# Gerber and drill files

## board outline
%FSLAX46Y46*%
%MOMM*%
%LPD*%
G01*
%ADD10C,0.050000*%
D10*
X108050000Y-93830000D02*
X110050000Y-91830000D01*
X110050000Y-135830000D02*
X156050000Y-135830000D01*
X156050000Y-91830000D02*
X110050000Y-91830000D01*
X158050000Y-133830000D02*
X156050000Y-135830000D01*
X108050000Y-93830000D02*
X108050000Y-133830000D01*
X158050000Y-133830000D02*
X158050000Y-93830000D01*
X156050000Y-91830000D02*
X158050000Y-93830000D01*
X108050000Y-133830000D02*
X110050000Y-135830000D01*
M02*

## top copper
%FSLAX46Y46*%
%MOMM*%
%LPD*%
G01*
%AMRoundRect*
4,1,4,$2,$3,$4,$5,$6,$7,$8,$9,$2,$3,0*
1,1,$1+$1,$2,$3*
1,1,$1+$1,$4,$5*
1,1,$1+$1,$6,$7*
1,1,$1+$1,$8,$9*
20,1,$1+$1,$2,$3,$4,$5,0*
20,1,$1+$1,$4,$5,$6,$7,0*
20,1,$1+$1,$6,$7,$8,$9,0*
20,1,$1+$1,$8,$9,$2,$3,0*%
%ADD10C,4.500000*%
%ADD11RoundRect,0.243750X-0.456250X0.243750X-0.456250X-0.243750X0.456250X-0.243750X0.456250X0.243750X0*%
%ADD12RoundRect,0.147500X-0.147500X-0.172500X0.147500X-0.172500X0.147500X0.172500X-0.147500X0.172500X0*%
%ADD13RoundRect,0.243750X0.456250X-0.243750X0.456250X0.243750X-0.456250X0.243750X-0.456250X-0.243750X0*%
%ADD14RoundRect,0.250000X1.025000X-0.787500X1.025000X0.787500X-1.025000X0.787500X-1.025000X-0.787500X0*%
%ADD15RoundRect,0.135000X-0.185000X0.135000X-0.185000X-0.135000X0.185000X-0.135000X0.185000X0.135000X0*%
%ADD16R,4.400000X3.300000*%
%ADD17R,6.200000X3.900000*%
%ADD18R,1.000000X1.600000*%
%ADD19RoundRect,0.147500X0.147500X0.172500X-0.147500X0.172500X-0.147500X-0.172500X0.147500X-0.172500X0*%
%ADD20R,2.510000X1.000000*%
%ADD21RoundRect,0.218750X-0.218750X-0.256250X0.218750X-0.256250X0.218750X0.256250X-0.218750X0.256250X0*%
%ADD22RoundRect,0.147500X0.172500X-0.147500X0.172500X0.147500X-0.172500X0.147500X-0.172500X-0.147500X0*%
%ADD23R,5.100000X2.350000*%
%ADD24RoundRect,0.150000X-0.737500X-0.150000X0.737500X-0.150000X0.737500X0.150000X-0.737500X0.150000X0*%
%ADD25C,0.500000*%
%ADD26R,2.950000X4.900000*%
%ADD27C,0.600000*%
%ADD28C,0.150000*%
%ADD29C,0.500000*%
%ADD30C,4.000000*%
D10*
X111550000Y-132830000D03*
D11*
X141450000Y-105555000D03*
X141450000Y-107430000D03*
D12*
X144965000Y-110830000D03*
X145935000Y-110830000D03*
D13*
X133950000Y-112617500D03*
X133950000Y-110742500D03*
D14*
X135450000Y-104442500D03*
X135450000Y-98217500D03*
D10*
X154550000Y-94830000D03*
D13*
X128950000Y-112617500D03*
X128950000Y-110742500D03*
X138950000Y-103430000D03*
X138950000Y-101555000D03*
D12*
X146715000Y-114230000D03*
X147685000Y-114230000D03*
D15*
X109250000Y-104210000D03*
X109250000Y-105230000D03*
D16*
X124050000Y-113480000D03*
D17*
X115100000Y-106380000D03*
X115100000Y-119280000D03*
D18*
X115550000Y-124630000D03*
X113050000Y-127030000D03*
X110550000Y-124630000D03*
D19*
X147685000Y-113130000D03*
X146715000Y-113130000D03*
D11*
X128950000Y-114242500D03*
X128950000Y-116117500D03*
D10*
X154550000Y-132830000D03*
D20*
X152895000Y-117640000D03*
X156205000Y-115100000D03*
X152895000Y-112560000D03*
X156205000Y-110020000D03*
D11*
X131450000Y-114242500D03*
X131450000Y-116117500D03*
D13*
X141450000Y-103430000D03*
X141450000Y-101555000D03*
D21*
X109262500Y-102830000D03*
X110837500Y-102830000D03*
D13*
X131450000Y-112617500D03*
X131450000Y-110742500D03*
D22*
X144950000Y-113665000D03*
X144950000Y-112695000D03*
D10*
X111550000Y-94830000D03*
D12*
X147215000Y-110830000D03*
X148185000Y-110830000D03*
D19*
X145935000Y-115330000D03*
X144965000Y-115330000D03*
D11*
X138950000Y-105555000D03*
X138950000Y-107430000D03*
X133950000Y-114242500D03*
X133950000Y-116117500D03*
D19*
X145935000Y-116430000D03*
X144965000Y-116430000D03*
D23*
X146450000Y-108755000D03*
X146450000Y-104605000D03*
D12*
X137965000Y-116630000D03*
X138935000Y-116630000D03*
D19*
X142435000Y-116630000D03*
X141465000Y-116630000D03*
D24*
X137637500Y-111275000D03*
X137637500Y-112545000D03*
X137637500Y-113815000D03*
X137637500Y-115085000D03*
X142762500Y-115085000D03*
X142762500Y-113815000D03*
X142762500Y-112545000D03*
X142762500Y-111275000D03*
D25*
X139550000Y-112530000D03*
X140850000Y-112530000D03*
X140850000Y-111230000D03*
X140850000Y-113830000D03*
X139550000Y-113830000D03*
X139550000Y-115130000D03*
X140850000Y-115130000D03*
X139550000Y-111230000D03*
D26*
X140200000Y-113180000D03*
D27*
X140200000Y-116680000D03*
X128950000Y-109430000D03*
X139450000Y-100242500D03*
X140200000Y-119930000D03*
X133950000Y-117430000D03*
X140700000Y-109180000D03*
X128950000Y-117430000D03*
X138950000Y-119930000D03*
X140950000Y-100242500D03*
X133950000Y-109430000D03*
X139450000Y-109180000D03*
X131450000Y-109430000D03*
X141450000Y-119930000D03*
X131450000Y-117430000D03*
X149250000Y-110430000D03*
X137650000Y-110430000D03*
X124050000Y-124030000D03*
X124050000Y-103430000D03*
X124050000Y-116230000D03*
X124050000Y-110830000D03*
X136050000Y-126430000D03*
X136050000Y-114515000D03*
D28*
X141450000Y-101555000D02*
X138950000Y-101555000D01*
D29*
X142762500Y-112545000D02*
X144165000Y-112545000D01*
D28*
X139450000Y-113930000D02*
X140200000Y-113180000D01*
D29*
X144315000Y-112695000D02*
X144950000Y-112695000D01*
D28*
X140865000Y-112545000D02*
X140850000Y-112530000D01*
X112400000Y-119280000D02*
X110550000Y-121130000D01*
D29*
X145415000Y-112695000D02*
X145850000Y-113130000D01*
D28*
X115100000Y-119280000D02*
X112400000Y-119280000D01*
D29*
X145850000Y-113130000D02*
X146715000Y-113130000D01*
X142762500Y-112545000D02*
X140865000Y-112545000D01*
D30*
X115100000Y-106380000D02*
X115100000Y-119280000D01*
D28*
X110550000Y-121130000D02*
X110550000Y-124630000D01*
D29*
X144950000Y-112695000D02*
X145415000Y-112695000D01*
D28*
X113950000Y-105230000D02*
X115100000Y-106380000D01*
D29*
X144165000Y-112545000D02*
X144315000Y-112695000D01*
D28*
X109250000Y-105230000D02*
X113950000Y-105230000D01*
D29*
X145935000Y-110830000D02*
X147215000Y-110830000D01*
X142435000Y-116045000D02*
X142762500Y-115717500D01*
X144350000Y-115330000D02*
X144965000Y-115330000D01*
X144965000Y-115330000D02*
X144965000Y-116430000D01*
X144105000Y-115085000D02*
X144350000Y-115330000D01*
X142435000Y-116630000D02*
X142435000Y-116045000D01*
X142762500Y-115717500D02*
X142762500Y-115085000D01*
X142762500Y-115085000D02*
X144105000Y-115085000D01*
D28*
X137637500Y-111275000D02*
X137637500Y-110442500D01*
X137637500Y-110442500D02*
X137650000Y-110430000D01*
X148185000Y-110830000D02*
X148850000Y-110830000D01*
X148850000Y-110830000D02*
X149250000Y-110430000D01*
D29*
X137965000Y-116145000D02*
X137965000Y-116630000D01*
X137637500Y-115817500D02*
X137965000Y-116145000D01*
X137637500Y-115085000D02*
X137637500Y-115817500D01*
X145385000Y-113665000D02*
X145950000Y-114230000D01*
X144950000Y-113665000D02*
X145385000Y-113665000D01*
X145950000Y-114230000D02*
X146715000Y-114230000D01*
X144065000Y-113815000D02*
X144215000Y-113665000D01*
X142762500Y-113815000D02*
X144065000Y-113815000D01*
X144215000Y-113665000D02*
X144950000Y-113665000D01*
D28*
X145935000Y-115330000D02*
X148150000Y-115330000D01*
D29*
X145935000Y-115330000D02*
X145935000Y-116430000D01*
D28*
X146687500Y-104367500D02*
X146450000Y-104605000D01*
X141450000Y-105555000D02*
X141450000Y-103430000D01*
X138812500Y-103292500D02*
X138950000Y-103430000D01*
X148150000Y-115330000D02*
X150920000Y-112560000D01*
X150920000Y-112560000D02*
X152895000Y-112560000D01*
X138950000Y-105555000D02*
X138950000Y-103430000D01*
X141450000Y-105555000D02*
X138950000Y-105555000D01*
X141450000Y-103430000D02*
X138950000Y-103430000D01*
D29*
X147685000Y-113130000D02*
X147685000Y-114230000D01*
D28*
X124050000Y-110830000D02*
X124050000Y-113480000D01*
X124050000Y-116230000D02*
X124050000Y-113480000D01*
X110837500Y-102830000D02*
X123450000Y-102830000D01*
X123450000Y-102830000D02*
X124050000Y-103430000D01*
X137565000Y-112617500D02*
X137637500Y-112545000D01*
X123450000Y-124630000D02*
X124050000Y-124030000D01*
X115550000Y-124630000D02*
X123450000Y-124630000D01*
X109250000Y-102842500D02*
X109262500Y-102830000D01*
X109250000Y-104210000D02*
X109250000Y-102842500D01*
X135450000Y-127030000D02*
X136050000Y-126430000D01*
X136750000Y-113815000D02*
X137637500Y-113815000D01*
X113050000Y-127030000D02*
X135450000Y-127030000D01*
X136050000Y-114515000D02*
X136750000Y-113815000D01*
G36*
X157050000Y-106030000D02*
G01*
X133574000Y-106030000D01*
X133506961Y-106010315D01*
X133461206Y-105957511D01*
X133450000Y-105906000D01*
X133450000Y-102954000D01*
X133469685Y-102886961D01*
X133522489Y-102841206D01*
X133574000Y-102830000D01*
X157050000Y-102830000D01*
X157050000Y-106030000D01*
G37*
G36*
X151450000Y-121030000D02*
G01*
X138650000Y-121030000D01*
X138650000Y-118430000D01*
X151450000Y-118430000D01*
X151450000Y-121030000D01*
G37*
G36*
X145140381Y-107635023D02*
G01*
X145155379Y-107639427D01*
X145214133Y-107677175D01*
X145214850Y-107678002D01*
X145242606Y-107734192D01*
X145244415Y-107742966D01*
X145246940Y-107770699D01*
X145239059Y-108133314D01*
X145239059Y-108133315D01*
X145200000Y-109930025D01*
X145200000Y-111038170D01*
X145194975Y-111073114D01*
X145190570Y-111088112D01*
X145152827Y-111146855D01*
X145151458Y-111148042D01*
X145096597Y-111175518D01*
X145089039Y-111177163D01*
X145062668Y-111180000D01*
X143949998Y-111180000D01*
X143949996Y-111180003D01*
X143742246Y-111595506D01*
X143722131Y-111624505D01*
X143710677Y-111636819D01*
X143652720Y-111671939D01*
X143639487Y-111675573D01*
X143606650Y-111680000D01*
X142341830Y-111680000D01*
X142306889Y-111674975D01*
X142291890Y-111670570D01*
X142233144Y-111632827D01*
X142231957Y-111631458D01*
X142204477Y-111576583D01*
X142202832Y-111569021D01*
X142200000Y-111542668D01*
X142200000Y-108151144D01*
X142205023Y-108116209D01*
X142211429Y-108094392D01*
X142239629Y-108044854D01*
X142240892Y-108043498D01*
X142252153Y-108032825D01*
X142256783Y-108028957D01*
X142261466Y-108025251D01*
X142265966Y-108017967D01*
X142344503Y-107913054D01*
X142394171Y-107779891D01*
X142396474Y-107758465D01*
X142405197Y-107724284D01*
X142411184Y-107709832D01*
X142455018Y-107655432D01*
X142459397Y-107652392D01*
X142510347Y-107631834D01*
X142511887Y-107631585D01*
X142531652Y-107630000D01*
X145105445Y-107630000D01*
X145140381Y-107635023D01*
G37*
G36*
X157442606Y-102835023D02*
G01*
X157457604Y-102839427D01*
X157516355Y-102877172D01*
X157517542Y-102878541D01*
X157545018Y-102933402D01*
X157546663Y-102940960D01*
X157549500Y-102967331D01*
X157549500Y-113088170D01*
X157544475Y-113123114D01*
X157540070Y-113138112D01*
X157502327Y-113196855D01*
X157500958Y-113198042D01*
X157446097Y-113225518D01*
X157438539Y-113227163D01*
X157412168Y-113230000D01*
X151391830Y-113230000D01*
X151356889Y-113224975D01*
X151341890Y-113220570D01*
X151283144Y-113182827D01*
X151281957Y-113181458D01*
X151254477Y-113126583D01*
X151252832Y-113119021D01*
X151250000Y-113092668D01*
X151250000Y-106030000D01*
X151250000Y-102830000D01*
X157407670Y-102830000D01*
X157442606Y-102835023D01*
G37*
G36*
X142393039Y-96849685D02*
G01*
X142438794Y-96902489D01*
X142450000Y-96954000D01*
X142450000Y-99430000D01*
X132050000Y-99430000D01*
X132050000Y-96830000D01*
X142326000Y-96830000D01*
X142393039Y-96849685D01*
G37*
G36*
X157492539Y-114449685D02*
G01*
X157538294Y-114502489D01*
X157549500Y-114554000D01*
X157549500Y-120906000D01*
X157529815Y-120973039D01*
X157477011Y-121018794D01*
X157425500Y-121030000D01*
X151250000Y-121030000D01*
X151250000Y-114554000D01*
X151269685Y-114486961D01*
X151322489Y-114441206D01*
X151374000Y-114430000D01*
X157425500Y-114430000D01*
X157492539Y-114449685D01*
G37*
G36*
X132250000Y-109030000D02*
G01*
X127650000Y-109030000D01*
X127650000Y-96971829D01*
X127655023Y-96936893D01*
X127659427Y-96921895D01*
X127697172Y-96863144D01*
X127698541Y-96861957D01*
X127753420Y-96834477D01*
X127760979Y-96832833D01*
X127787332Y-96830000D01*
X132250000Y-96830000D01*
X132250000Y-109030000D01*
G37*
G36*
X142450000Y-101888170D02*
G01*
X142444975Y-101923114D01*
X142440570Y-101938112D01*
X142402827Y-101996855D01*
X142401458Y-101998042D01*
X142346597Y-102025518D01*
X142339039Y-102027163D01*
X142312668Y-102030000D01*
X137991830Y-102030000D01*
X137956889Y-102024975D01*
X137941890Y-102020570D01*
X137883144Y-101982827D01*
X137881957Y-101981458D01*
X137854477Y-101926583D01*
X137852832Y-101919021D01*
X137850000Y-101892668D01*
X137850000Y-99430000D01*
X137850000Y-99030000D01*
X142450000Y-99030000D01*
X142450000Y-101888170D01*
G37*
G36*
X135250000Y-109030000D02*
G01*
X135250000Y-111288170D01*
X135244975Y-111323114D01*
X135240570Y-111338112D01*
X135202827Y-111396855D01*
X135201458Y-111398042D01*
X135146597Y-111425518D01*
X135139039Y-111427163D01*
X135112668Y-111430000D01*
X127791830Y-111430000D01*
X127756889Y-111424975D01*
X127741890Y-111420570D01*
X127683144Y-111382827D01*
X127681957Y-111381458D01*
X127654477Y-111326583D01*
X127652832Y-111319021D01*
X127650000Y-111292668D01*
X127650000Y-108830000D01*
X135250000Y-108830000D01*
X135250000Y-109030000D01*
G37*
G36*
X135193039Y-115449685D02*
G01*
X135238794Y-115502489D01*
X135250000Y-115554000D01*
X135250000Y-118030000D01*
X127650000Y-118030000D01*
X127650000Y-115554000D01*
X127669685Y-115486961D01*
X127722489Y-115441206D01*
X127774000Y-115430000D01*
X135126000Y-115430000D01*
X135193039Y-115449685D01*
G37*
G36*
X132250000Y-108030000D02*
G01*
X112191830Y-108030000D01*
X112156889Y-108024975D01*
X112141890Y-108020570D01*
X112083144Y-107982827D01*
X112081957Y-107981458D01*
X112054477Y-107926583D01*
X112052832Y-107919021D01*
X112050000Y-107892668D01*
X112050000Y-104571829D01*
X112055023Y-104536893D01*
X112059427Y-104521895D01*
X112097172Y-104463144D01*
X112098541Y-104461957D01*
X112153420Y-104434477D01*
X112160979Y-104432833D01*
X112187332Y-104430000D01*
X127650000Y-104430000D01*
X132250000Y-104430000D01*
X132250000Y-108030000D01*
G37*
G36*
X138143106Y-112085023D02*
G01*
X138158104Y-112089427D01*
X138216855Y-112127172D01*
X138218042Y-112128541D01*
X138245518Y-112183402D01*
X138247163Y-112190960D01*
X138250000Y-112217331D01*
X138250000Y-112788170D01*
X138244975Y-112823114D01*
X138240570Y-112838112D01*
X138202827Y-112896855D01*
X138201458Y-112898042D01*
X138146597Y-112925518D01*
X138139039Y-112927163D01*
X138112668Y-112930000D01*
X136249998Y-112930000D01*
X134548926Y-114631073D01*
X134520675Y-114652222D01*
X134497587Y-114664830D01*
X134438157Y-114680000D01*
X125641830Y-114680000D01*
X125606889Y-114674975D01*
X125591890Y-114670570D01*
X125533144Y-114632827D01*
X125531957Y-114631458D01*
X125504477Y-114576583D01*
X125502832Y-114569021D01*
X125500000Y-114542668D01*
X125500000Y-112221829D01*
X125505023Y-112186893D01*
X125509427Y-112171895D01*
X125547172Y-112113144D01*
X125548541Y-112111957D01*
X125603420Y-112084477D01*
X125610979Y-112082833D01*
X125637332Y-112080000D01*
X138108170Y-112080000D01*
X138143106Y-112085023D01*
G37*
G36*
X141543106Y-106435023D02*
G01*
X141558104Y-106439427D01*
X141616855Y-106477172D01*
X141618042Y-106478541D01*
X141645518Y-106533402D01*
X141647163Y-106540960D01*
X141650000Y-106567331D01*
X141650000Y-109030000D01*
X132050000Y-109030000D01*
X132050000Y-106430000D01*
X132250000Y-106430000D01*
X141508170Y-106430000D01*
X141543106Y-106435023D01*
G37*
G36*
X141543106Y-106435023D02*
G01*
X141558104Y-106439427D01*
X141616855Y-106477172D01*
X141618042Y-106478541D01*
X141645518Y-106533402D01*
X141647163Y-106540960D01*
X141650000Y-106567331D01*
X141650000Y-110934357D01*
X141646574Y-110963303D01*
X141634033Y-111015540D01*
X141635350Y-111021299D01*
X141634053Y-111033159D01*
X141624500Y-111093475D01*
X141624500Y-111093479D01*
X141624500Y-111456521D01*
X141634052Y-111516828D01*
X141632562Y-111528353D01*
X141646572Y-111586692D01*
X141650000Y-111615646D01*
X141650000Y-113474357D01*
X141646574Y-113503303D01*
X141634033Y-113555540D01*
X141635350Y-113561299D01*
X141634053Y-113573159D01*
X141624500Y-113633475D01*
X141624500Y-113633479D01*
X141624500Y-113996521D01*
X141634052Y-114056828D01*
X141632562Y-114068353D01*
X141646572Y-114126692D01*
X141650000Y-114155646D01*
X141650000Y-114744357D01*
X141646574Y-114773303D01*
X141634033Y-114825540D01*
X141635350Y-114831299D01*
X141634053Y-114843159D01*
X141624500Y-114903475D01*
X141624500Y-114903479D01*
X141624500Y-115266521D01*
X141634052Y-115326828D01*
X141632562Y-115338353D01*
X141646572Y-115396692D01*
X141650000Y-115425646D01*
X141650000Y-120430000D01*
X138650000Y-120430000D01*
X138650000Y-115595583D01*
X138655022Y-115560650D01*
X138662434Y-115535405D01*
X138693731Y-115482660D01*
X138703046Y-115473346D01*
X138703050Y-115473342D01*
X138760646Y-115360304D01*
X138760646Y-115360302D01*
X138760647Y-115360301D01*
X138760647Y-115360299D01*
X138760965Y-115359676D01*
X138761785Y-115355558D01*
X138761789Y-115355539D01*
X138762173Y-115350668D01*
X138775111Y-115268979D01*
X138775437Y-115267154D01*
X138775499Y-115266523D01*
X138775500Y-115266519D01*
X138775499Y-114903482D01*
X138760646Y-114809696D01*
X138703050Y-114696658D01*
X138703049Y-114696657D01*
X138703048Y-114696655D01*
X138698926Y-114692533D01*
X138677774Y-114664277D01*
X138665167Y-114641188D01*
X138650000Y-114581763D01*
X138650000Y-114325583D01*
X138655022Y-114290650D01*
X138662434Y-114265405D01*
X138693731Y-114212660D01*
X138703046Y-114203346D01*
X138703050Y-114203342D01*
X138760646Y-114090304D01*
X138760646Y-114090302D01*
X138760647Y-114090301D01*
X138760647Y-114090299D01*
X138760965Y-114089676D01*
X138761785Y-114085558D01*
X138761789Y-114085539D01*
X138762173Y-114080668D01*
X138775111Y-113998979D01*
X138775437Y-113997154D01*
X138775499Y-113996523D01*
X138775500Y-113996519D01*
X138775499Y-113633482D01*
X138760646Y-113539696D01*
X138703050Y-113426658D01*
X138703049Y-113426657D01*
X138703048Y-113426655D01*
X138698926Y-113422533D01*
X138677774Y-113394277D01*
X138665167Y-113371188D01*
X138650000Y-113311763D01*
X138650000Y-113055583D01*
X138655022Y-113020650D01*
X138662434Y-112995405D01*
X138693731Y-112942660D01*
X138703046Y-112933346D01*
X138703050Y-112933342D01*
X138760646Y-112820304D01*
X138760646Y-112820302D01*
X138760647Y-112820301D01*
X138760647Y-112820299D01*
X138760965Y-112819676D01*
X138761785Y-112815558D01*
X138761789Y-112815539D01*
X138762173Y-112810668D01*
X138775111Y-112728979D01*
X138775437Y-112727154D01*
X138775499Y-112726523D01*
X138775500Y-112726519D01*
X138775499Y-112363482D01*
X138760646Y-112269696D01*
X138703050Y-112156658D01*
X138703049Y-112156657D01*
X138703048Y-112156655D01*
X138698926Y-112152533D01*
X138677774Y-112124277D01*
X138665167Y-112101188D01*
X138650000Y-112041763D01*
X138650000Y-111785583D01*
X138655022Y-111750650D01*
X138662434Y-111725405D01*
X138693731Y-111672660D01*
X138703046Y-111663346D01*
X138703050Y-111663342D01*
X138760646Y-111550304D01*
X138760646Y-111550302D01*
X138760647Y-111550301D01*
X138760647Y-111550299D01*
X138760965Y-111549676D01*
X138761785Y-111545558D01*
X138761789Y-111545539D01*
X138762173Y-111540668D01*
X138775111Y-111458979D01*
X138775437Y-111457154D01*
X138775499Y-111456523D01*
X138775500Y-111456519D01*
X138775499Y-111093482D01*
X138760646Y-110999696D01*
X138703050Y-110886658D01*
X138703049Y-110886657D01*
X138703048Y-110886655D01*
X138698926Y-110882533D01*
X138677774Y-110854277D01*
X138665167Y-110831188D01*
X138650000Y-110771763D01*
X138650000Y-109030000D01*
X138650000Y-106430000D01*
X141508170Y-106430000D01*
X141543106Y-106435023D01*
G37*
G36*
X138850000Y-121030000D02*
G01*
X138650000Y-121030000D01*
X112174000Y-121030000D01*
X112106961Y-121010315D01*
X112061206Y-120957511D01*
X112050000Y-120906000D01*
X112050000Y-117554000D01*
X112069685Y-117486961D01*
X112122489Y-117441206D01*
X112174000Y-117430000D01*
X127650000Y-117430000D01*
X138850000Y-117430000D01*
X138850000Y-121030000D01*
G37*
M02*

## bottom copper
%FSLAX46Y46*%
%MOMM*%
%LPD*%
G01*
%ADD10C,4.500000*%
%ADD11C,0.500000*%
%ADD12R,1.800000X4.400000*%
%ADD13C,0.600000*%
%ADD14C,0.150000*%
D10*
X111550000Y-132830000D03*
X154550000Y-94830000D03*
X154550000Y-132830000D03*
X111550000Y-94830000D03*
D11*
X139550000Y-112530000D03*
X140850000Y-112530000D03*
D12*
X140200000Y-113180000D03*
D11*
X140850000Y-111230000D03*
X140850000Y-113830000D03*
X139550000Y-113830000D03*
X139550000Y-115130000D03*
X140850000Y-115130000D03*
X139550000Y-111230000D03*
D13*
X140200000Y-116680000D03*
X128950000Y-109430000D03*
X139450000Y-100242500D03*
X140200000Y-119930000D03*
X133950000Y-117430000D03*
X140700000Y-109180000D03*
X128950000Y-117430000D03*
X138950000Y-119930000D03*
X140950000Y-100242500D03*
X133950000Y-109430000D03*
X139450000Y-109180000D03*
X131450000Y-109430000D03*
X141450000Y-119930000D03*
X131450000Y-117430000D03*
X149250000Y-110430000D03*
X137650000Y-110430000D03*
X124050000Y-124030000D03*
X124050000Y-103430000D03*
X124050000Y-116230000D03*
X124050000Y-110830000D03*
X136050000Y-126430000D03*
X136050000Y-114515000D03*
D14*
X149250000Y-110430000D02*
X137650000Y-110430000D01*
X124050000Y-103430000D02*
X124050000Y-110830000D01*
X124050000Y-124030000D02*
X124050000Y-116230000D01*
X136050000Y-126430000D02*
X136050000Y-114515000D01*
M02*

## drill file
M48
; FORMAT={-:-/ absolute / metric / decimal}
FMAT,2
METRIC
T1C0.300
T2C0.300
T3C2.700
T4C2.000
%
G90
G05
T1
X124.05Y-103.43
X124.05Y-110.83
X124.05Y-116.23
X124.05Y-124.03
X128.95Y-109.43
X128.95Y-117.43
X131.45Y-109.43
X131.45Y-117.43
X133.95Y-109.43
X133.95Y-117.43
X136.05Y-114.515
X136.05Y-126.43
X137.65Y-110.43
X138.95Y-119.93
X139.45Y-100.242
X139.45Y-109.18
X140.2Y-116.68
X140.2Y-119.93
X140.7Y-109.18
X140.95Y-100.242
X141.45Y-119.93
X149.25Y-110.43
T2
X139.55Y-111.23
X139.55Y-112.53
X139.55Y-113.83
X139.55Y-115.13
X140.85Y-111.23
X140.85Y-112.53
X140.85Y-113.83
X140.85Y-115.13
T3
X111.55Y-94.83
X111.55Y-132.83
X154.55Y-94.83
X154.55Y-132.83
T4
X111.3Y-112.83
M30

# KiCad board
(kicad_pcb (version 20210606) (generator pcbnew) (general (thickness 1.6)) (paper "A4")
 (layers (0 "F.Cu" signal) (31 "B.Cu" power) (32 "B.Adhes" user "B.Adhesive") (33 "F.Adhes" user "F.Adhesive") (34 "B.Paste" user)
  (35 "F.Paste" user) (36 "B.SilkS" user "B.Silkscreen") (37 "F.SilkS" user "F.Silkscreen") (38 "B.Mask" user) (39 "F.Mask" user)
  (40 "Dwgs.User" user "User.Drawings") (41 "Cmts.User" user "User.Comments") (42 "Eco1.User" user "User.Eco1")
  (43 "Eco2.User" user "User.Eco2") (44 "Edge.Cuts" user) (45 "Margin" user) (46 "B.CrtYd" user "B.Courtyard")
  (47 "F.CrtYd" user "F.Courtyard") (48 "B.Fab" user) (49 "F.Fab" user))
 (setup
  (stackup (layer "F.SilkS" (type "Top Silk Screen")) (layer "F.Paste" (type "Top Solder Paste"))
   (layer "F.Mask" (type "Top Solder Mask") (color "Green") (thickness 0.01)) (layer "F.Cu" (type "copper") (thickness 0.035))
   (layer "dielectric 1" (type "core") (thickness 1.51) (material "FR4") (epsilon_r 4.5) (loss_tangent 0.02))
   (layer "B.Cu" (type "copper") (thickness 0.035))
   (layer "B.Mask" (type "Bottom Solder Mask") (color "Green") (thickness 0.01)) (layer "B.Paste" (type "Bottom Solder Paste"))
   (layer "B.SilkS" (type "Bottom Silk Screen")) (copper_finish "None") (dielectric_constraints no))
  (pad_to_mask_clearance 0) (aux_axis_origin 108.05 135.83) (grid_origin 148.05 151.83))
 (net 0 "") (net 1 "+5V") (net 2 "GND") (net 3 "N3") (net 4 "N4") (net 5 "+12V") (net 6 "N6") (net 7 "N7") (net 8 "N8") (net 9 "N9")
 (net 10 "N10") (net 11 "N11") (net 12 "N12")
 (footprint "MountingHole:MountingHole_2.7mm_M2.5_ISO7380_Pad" (layer "F.Cu") (at 111.55 132.83)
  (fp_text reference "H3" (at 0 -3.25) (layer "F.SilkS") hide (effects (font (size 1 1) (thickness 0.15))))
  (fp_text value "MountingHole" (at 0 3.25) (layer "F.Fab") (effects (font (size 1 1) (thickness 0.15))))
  (pad "1" thru_hole circle locked (at 0 0) (size 4.5 4.5) (drill 2.7) (layers *.Cu *.Mask)))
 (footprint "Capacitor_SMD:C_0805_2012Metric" (layer "F.Cu") (at 141.45 106.4925 -90)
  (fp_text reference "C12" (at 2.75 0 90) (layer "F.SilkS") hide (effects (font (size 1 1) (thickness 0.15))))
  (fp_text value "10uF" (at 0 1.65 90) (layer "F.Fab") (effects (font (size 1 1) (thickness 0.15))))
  (pad "1" smd roundrect locked (at -0.9375 0 270) (size 0.975 1.4) (layers "F.Cu" "F.Paste" "F.Mask") (roundrect_rratio 0.25) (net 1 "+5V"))
  (pad "2" smd roundrect locked (at 0.9375 0 270) (size 0.975 1.4) (layers "F.Cu" "F.Paste" "F.Mask") (roundrect_rratio 0.25) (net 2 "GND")))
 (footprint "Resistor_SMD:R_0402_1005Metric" (layer "F.Cu") (at 145.45 110.83)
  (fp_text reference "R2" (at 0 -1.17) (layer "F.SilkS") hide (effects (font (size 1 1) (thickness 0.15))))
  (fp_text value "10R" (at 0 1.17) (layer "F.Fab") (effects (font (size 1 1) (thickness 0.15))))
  (pad "1" smd roundrect locked (at -0.485 0) (size 0.59 0.64) (layers "F.Cu" "F.Paste" "F.Mask") (roundrect_rratio 0.25) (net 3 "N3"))
  (pad "2" smd roundrect locked (at 0.485 0) (size 0.59 0.64) (layers "F.Cu" "F.Paste" "F.Mask") (roundrect_rratio 0.25) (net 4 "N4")))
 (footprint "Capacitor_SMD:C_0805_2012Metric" (layer "F.Cu") (at 133.95 111.68 90)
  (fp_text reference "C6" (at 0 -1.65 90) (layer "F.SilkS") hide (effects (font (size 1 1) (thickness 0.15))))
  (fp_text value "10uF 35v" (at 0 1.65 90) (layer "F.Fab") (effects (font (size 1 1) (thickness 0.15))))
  (pad "1" smd roundrect locked (at -0.9375 0 90) (size 0.975 1.4) (layers "F.Cu" "F.Paste" "F.Mask") (roundrect_rratio 0.25) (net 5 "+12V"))
  (pad "2" smd roundrect locked (at 0.9375 0 90) (size 0.975 1.4) (layers "F.Cu" "F.Paste" "F.Mask") (roundrect_rratio 0.25) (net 2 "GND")))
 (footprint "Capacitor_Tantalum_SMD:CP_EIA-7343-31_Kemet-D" (layer "F.Cu") (at 135.45 101.33 90)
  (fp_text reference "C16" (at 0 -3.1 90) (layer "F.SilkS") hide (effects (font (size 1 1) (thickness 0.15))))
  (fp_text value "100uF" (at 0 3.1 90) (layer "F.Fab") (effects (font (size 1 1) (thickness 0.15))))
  (pad "1" smd roundrect locked (at -3.1125 0 90) (size 2.075 2.55) (layers "F.Cu" "F.Paste" "F.Mask") (roundrect_rratio 0.1204819277)
   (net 1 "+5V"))
  (pad "2" smd roundrect locked (at 3.1125 0 90) (size 2.075 2.55) (layers "F.Cu" "F.Paste" "F.Mask") (roundrect_rratio 0.1204819277)
   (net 2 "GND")))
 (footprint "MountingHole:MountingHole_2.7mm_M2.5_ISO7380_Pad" (layer "F.Cu") (at 154.55 94.83)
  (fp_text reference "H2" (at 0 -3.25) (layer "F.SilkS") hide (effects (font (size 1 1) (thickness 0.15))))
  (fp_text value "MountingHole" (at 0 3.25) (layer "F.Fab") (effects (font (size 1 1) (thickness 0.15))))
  (pad "1" thru_hole circle locked (at 0 0) (size 4.5 4.5) (drill 2.7) (layers *.Cu *.Mask)))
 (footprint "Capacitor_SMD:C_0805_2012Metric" (layer "F.Cu") (at 128.95 111.68 90)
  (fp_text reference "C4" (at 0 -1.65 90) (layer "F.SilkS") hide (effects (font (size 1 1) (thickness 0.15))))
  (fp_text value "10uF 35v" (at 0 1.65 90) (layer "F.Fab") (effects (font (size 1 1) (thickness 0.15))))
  (pad "1" smd roundrect locked (at -0.9375 0 90) (size 0.975 1.4) (layers "F.Cu" "F.Paste" "F.Mask") (roundrect_rratio 0.25) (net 5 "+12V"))
  (pad "2" smd roundrect locked (at 0.9375 0 90) (size 0.975 1.4) (layers "F.Cu" "F.Paste" "F.Mask") (roundrect_rratio 0.25) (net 2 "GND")))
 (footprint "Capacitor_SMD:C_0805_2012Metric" (layer "F.Cu") (at 138.95 102.4925 90)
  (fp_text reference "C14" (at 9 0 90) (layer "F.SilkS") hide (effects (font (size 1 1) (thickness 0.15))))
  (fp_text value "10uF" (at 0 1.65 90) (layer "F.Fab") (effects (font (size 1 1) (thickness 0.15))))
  (pad "1" smd roundrect locked (at -0.9375 0 90) (size 0.975 1.4) (layers "F.Cu" "F.Paste" "F.Mask") (roundrect_rratio 0.25) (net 1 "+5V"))
  (pad "2" smd roundrect locked (at 0.9375 0 90) (size 0.975 1.4) (layers "F.Cu" "F.Paste" "F.Mask") (roundrect_rratio 0.25) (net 2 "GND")))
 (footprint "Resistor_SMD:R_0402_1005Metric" (layer "F.Cu") (at 147.2 114.23)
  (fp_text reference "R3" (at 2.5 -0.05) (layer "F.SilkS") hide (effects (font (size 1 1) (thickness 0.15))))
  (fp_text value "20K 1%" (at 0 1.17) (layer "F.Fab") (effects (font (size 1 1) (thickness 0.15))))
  (pad "1" smd roundrect locked (at -0.485 0) (size 0.59 0.64) (layers "F.Cu" "F.Paste" "F.Mask") (roundrect_rratio 0.25) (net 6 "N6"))
  (pad "2" smd roundrect locked (at 0.485 0) (size 0.59 0.64) (layers "F.Cu" "F.Paste" "F.Mask") (roundrect_rratio 0.25) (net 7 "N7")))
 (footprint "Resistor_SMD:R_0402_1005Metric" (layer "F.Cu") (at 109.25 104.72 -90)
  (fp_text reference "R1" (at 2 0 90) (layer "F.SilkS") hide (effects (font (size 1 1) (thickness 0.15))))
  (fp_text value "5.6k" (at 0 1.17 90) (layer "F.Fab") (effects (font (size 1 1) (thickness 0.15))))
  (pad "1" smd roundrect locked (at -0.51 0 270) (size 0.54 0.64) (layers "F.Cu" "F.Paste" "F.Mask") (roundrect_rratio 0.25) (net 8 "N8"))
  (pad "2" smd roundrect locked (at 0.51 0 270) (size 0.54 0.64) (layers "F.Cu" "F.Paste" "F.Mask") (roundrect_rratio 0.25) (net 2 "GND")))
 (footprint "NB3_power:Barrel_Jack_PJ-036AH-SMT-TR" (layer "F.Cu") (at 124.05 113.48)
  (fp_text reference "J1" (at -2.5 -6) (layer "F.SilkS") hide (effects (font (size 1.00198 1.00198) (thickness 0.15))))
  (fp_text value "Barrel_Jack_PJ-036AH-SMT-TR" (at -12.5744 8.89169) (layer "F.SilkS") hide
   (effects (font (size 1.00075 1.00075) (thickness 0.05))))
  (pad "1" smd rect locked (at 0 0 90) (size 3.3 4.4) (layers "F.Cu" "F.Paste" "F.Mask") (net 5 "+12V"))
  (pad "2" smd rect locked (at -8.95 -7.1 180) (size 6.2 3.9) (layers "F.Cu" "F.Paste" "F.Mask") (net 2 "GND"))
  (pad "3" smd rect locked (at -8.95 5.8) (size 6.2 3.9) (layers "F.Cu" "F.Paste" "F.Mask") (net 2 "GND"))
  (pad "Hole" np_thru_hole circle locked (at -12.75 -0.65) (size 2 2) (drill 2) (layers *.Cu *.Mask "F.SilkS")))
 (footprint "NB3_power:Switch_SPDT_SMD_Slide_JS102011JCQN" (layer "F.Cu") (at 113.05 125.83 180)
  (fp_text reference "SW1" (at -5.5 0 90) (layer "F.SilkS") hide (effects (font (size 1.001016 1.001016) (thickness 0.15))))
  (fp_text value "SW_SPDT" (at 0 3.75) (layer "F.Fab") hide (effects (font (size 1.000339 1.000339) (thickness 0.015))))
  (pad "1" smd rect locked (at -2.5 1.2 180) (size 1 1.6) (layers "F.Cu" "F.Paste" "F.Mask") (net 5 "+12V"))
  (pad "2" smd rect locked (at 0 -1.2 180) (size 1 1.6) (layers "F.Cu" "F.Paste" "F.Mask") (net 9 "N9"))
  (pad "3" smd rect locked (at 2.5 1.2 180) (size 1 1.6) (layers "F.Cu" "F.Paste" "F.Mask") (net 2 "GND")))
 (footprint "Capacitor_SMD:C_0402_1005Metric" (layer "F.Cu") (at 147.2 113.13 180)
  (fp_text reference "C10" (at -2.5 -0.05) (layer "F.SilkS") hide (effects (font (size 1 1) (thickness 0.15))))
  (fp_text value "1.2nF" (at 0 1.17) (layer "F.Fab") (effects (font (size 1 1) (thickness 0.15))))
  (pad "1" smd roundrect locked (at -0.485 0 180) (size 0.59 0.64) (layers "F.Cu" "F.Paste" "F.Mask") (roundrect_rratio 0.25) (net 7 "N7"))
  (pad "2" smd roundrect locked (at 0.485 0 180) (size 0.59 0.64) (layers "F.Cu" "F.Paste" "F.Mask") (roundrect_rratio 0.25) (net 2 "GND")))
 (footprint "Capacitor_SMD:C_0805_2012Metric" (layer "F.Cu") (at 128.95 115.18 -90)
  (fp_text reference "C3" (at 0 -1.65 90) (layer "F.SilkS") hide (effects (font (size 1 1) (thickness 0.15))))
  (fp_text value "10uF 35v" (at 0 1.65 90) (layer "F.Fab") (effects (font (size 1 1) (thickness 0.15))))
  (pad "1" smd roundrect locked (at -0.9375 0 270) (size 0.975 1.4) (layers "F.Cu" "F.Paste" "F.Mask") (roundrect_rratio 0.25)
   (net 5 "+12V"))
  (pad "2" smd roundrect locked (at 0.9375 0 270) (size 0.975 1.4) (layers "F.Cu" "F.Paste" "F.Mask") (roundrect_rratio 0.25) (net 2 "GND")))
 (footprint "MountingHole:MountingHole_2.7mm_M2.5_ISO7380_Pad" (layer "F.Cu") (at 154.55 132.83)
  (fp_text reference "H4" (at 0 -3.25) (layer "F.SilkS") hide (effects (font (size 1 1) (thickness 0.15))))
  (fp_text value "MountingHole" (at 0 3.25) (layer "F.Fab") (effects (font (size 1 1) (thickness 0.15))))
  (pad "1" thru_hole circle locked (at 0 0) (size 4.5 4.5) (drill 2.7) (layers *.Cu *.Mask)))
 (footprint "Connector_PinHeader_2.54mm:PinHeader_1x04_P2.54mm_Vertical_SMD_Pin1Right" (layer "F.Cu") (at 154.55 113.83 180)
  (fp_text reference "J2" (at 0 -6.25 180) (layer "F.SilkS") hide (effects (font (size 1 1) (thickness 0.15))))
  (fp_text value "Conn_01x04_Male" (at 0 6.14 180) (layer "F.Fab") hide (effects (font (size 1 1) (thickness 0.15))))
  (pad "1" smd rect locked (at 1.655 -3.81 180) (size 2.51 1) (layers "F.Cu" "F.Paste" "F.Mask") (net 2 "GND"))
  (pad "2" smd rect locked (at -1.655 -1.27 180) (size 2.51 1) (layers "F.Cu" "F.Paste" "F.Mask") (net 2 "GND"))
  (pad "3" smd rect locked (at 1.655 1.27 180) (size 2.51 1) (layers "F.Cu" "F.Paste" "F.Mask") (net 1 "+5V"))
  (pad "4" smd rect locked (at -1.655 3.81 180) (size 2.51 1) (layers "F.Cu" "F.Paste" "F.Mask") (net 1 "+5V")))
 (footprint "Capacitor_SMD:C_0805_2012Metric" (layer "F.Cu") (at 131.45 115.18 -90)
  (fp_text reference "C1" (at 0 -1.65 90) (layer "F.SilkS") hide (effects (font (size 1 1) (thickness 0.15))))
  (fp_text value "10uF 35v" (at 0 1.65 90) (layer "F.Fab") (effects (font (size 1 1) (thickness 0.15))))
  (pad "1" smd roundrect locked (at -0.9375 0 270) (size 0.975 1.4) (layers "F.Cu" "F.Paste" "F.Mask") (roundrect_rratio 0.25)
   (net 5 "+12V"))
  (pad "2" smd roundrect locked (at 0.9375 0 270) (size 0.975 1.4) (layers "F.Cu" "F.Paste" "F.Mask") (roundrect_rratio 0.25) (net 2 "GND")))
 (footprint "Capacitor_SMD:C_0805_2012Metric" (layer "F.Cu") (at 141.45 102.4925 90)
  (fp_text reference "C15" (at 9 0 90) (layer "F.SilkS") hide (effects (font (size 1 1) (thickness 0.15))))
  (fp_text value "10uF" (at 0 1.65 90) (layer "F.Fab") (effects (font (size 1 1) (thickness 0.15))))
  (pad "1" smd roundrect locked (at -0.9375 0 90) (size 0.975 1.4) (layers "F.Cu" "F.Paste" "F.Mask") (roundrect_rratio 0.25) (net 1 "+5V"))
  (pad "2" smd roundrect locked (at 0.9375 0 90) (size 0.975 1.4) (layers "F.Cu" "F.Paste" "F.Mask") (roundrect_rratio 0.25) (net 2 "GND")))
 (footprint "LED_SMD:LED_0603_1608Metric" (layer "F.Cu") (at 110.05 102.83)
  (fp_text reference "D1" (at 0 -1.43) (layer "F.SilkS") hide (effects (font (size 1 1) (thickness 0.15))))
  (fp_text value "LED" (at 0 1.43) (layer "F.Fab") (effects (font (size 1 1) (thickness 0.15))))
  (pad "1" smd roundrect locked (at -0.7875 0) (size 0.875 0.95) (layers "F.Cu" "F.Paste" "F.Mask") (roundrect_rratio 0.25) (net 8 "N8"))
  (pad "2" smd roundrect locked (at 0.7875 0) (size 0.875 0.95) (layers "F.Cu" "F.Paste" "F.Mask") (roundrect_rratio 0.25) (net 5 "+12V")))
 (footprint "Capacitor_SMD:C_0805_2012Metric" (layer "F.Cu") (at 131.45 111.68 90)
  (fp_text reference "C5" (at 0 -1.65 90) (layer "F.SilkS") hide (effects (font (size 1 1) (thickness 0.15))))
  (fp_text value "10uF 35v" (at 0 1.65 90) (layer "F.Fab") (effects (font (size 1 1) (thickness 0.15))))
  (pad "1" smd roundrect locked (at -0.9375 0 90) (size 0.975 1.4) (layers "F.Cu" "F.Paste" "F.Mask") (roundrect_rratio 0.25) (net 5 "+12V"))
  (pad "2" smd roundrect locked (at 0.9375 0 90) (size 0.975 1.4) (layers "F.Cu" "F.Paste" "F.Mask") (roundrect_rratio 0.25) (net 2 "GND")))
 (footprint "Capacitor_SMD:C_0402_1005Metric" (layer "F.Cu") (at 144.95 113.18 90)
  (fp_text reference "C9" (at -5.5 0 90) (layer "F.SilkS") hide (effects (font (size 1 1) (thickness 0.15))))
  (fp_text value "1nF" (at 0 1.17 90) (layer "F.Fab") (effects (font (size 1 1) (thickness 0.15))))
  (pad "1" smd roundrect locked (at -0.485 0 90) (size 0.59 0.64) (layers "F.Cu" "F.Paste" "F.Mask") (roundrect_rratio 0.25) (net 6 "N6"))
  (pad "2" smd roundrect locked (at 0.485 0 90) (size 0.59 0.64) (layers "F.Cu" "F.Paste" "F.Mask") (roundrect_rratio 0.25) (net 2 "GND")))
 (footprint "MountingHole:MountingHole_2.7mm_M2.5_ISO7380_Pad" (layer "F.Cu") (at 111.55 94.83)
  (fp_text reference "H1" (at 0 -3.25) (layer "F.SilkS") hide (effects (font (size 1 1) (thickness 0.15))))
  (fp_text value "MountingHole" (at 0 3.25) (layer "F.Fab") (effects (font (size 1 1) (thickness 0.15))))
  (pad "1" thru_hole circle locked (at 0 0) (size 4.5 4.5) (drill 2.7) (layers *.Cu *.Mask)))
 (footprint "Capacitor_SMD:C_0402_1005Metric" (layer "F.Cu") (at 147.7 110.83)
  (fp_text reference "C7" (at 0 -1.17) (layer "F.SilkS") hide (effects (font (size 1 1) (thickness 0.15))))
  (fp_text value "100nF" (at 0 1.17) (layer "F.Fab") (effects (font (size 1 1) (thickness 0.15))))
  (pad "1" smd roundrect locked (at -0.485 0) (size 0.59 0.64) (layers "F.Cu" "F.Paste" "F.Mask") (roundrect_rratio 0.25) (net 4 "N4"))
  (pad "2" smd roundrect locked (at 0.485 0) (size 0.59 0.64) (layers "F.Cu" "F.Paste" "F.Mask") (roundrect_rratio 0.25) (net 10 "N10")))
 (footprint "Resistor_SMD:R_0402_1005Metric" (layer "F.Cu") (at 145.45 115.33 180)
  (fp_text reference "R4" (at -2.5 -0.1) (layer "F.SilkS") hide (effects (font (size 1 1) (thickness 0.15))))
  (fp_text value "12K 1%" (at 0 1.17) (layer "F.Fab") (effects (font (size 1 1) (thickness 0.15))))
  (pad "1" smd roundrect locked (at -0.485 0 180) (size 0.59 0.64) (layers "F.Cu" "F.Paste" "F.Mask") (roundrect_rratio 0.25) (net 1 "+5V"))
  (pad "2" smd roundrect locked (at 0.485 0 180) (size 0.59 0.64) (layers "F.Cu" "F.Paste" "F.Mask") (roundrect_rratio 0.25) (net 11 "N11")))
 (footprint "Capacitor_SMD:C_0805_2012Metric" (layer "F.Cu") (at 138.95 106.4925 -90)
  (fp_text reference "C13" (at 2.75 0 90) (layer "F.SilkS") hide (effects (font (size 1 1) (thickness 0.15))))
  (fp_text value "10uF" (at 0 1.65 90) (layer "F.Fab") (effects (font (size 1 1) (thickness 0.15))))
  (pad "1" smd roundrect locked (at -0.9375 0 270) (size 0.975 1.4) (layers "F.Cu" "F.Paste" "F.Mask") (roundrect_rratio 0.25) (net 1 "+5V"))
  (pad "2" smd roundrect locked (at 0.9375 0 270) (size 0.975 1.4) (layers "F.Cu" "F.Paste" "F.Mask") (roundrect_rratio 0.25) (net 2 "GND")))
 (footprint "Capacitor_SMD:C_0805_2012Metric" (layer "F.Cu") (at 133.95 115.18 -90)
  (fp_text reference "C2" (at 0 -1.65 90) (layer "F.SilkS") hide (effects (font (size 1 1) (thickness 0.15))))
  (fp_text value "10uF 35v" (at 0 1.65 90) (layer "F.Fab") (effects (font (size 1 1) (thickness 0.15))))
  (pad "1" smd roundrect locked (at -0.9375 0 270) (size 0.975 1.4) (layers "F.Cu" "F.Paste" "F.Mask") (roundrect_rratio 0.25)
   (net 5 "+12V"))
  (pad "2" smd roundrect locked (at 0.9375 0 270) (size 0.975 1.4) (layers "F.Cu" "F.Paste" "F.Mask") (roundrect_rratio 0.25) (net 2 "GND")))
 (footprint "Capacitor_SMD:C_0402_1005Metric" (layer "F.Cu") (at 145.45 116.43 180)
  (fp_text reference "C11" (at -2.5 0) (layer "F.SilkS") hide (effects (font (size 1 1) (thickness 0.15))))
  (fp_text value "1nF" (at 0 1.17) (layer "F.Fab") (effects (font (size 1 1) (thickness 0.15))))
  (pad "1" smd roundrect locked (at -0.485 0 180) (size 0.59 0.64) (layers "F.Cu" "F.Paste" "F.Mask") (roundrect_rratio 0.25) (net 1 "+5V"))
  (pad "2" smd roundrect locked (at 0.485 0 180) (size 0.59 0.64) (layers "F.Cu" "F.Paste" "F.Mask") (roundrect_rratio 0.25) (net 11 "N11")))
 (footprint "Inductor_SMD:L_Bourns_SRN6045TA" (layer "F.Cu") (at 146.45 106.68 90)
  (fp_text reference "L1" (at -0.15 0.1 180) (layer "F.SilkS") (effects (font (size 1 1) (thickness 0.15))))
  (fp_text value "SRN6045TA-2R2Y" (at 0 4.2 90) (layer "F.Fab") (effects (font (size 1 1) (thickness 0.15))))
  (pad "1" smd rect locked (at -2.075 0 90) (size 2.35 5.1) (layers "F.Cu" "F.Paste" "F.Mask") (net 3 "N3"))
  (pad "2" smd rect locked (at 2.075 0 90) (size 2.35 5.1) (layers "F.Cu" "F.Paste" "F.Mask") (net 1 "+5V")))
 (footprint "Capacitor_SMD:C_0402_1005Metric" (layer "F.Cu") (at 138.45 116.63)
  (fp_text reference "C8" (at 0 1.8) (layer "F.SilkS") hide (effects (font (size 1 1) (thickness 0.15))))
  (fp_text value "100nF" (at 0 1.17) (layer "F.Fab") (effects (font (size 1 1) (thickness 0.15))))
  (pad "1" smd roundrect locked (at -0.485 0) (size 0.59 0.64) (layers "F.Cu" "F.Paste" "F.Mask") (roundrect_rratio 0.25) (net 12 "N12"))
  (pad "2" smd roundrect locked (at 0.485 0) (size 0.59 0.64) (layers "F.Cu" "F.Paste" "F.Mask") (roundrect_rratio 0.25) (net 2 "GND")))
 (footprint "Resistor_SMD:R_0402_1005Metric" (layer "F.Cu") (at 141.95 116.63 180)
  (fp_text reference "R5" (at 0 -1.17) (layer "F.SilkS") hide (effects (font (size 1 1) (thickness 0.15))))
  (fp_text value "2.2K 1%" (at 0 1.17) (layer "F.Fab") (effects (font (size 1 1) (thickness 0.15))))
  (pad "1" smd roundrect locked (at -0.485 0 180) (size 0.59 0.64) (layers "F.Cu" "F.Paste" "F.Mask") (roundrect_rratio 0.25) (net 11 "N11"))
  (pad "2" smd roundrect locked (at 0.485 0 180) (size 0.59 0.64) (layers "F.Cu" "F.Paste" "F.Mask") (roundrect_rratio 0.25) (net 2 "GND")))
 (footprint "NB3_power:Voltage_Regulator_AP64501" (layer "F.Cu") (at 140.2 113.18)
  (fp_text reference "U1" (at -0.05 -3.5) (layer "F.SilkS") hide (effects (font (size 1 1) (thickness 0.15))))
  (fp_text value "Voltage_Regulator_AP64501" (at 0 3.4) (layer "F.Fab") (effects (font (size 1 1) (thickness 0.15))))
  (pad "" smd roundrect locked (at 0.68 0.85) (size 1.13 1.42) (layers "F.Paste") (roundrect_rratio 0.2212389381))
  (pad "" smd rect locked (at 0 0) (size 2.71 3.4) (layers "F.Mask"))
  (pad "" smd roundrect locked (at -0.68 -0.85) (size 1.13 1.42) (layers "F.Paste") (roundrect_rratio 0.2212389381))
  (pad "" smd roundrect locked (at -0.68 0.85) (size 1.13 1.42) (layers "F.Paste") (roundrect_rratio 0.2212389381))
  (pad "" smd roundrect locked (at 0.68 -0.85) (size 1.13 1.42) (layers "F.Paste") (roundrect_rratio 0.2212389381))
  (pad "1" smd roundrect locked (at -2.5625 -1.905) (size 1.775 0.6) (layers "F.Cu" "F.Paste" "F.Mask") (roundrect_rratio 0.25)
   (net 10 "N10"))
  (pad "2" smd roundrect locked (at -2.5625 -0.635) (size 1.775 0.6) (layers "F.Cu" "F.Paste" "F.Mask") (roundrect_rratio 0.25)
   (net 5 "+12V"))
  (pad "3" smd roundrect locked (at -2.5625 0.635) (size 1.775 0.6) (layers "F.Cu" "F.Paste" "F.Mask") (roundrect_rratio 0.25) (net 9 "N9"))
  (pad "4" smd roundrect locked (at -2.5625 1.905) (size 1.775 0.6) (layers "F.Cu" "F.Paste" "F.Mask") (roundrect_rratio 0.25)
   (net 12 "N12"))
  (pad "5" smd roundrect locked (at 2.5625 1.905) (size 1.775 0.6) (layers "F.Cu" "F.Paste" "F.Mask") (roundrect_rratio 0.25) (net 11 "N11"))
  (pad "6" smd roundrect locked (at 2.5625 0.635) (size 1.775 0.6) (layers "F.Cu" "F.Paste" "F.Mask") (roundrect_rratio 0.25) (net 6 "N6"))
  (pad "7" smd roundrect locked (at 2.5625 -0.635) (size 1.775 0.6) (layers "F.Cu" "F.Paste" "F.Mask") (roundrect_rratio 0.25) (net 2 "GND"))
  (pad "8" smd roundrect locked (at 2.5625 -1.905) (size 1.775 0.6) (layers "F.Cu" "F.Paste" "F.Mask") (roundrect_rratio 0.25) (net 3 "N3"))
  (pad "9" thru_hole circle locked (at -0.65 -0.65) (size 0.5 0.5) (drill 0.3) (layers *.Cu) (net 2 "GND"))
  (pad "9" thru_hole circle locked (at 0.65 -0.65) (size 0.5 0.5) (drill 0.3) (layers *.Cu) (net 2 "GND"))
  (pad "9" smd rect locked (at 0 0) (size 1.8 4.4) (layers "B.Cu" "B.Mask") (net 2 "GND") (solder_mask_margin 0.1))
  (pad "9" thru_hole circle locked (at 0.65 -1.95) (size 0.5 0.5) (drill 0.3) (layers *.Cu) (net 2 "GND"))
  (pad "9" thru_hole circle locked (at 0.65 0.65) (size 0.5 0.5) (drill 0.3) (layers *.Cu) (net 2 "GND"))
  (pad "9" thru_hole circle locked (at -0.65 0.65 270) (size 0.5 0.5) (drill 0.3) (layers *.Cu) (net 2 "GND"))
  (pad "9" thru_hole circle locked (at -0.65 1.95) (size 0.5 0.5) (drill 0.3) (layers *.Cu) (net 2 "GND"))
  (pad "9" thru_hole circle locked (at 0.65 1.95) (size 0.5 0.5) (drill 0.3) (layers *.Cu) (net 2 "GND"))
  (pad "9" thru_hole circle locked (at -0.65 -1.95) (size 0.5 0.5) (drill 0.3) (layers *.Cu) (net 2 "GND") (solder_mask_margin 0.3))
  (pad "9" smd rect locked (at 0 0) (size 2.95 4.9) (layers "F.Cu") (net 2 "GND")))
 (gr_line (start 108.05 93.83) (end 110.05 91.83) (layer "Edge.Cuts") (width 0.05))
 (gr_line (start 110.05 135.83) (end 156.05 135.83) (layer "Edge.Cuts") (width 0.05))
 (gr_line (start 156.05 91.83) (end 110.05 91.83) (layer "Edge.Cuts") (width 0.05))
 (gr_line (start 158.05 133.83) (end 156.05 135.83) (layer "Edge.Cuts") (width 0.05))
 (gr_line (start 108.05 93.83) (end 108.05 133.83) (layer "Edge.Cuts") (width 0.05))
 (gr_line (start 158.05 133.83) (end 158.05 93.83) (layer "Edge.Cuts") (width 0.05))
 (gr_line (start 156.05 91.83) (end 158.05 93.83) (layer "Edge.Cuts") (width 0.05))
 (gr_line (start 108.05 133.83) (end 110.05 135.83) (layer "Edge.Cuts") (width 0.05))
 (segment (start 141.45 101.555) (end 138.95 101.555) (width 0.15) (layer "F.Cu") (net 2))
 (segment (start 142.7625 112.545) (end 144.165 112.545) (width 0.5) (layer "F.Cu") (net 2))
 (segment (start 139.45 113.93) (end 140.2 113.18) (width 0.15) (layer "F.Cu") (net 2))
 (segment (start 144.315 112.695) (end 144.95 112.695) (width 0.5) (layer "F.Cu") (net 2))
 (segment (start 140.865 112.545) (end 140.85 112.53) (width 0.15) (layer "F.Cu") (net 2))
 (segment (start 112.4 119.28) (end 110.55 121.13) (width 0.15) (layer "F.Cu") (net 2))
 (segment (start 145.415 112.695) (end 145.85 113.13) (width 0.5) (layer "F.Cu") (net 2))
 (segment (start 115.1 119.28) (end 112.4 119.28) (width 0.15) (layer "F.Cu") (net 2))
 (segment (start 145.85 113.13) (end 146.715 113.13) (width 0.5) (layer "F.Cu") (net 2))
 (segment (start 142.7625 112.545) (end 140.865 112.545) (width 0.5) (layer "F.Cu") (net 2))
 (segment (start 115.1 106.38) (end 115.1 119.28) (width 4) (layer "F.Cu") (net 2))
 (segment (start 110.55 121.13) (end 110.55 124.63) (width 0.15) (layer "F.Cu") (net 2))
 (segment (start 144.95 112.695) (end 145.415 112.695) (width 0.5) (layer "F.Cu") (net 2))
 (segment (start 113.95 105.23) (end 115.1 106.38) (width 0.15) (layer "F.Cu") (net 2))
 (segment (start 144.165 112.545) (end 144.315 112.695) (width 0.5) (layer "F.Cu") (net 2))
 (segment (start 109.25 105.23) (end 113.95 105.23) (width 0.15) (layer "F.Cu") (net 2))
 (via (at 140.2 116.68) (size 0.6) (drill 0.3) (layers "F.Cu" "B.Cu") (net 2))
 (via (at 128.95 109.43) (size 0.6) (drill 0.3) (layers "F.Cu" "B.Cu") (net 2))
 (via (at 139.45 100.2425) (size 0.6) (drill 0.3) (layers "F.Cu" "B.Cu") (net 2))
 (via (at 140.2 119.93) (size 0.6) (drill 0.3) (layers "F.Cu" "B.Cu") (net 2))
 (via (at 133.95 117.43) (size 0.6) (drill 0.3) (layers "F.Cu" "B.Cu") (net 2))
 (via (at 140.7 109.18) (size 0.6) (drill 0.3) (layers "F.Cu" "B.Cu") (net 2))
 (via (at 128.95 117.43) (size 0.6) (drill 0.3) (layers "F.Cu" "B.Cu") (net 2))
 (via (at 138.95 119.93) (size 0.6) (drill 0.3) (layers "F.Cu" "B.Cu") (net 2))
 (via (at 140.95 100.2425) (size 0.6) (drill 0.3) (layers "F.Cu" "B.Cu") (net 2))
 (via (at 133.95 109.43) (size 0.6) (drill 0.3) (layers "F.Cu" "B.Cu") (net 2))
 (via (at 139.45 109.18) (size 0.6) (drill 0.3) (layers "F.Cu" "B.Cu") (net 2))
 (via (at 131.45 109.43) (size 0.6) (drill 0.3) (layers "F.Cu" "B.Cu") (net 2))
 (via (at 141.45 119.93) (size 0.6) (drill 0.3) (layers "F.Cu" "B.Cu") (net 2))
 (via (at 131.45 117.43) (size 0.6) (drill 0.3) (layers "F.Cu" "B.Cu") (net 2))
 (segment (start 145.935 110.83) (end 147.215 110.83) (width 0.5) (layer "F.Cu") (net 4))
 (segment (start 142.435 116.045) (end 142.7625 115.7175) (width 0.5) (layer "F.Cu") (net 11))
 (segment (start 144.35 115.33) (end 144.965 115.33) (width 0.5) (layer "F.Cu") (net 11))
 (segment (start 144.965 115.33) (end 144.965 116.43) (width 0.5) (layer "F.Cu") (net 11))
 (segment (start 144.105 115.085) (end 144.35 115.33) (width 0.5) (layer "F.Cu") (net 11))
 (segment (start 142.435 116.63) (end 142.435 116.045) (width 0.5) (layer "F.Cu") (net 11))
 (segment (start 142.7625 115.7175) (end 142.7625 115.085) (width 0.5) (layer "F.Cu") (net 11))
 (segment (start 142.7625 115.085) (end 144.105 115.085) (width 0.5) (layer "F.Cu") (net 11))
 (segment (start 137.6375 111.275) (end 137.6375 110.4425) (width 0.15) (layer "F.Cu") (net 10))
 (segment (start 137.6375 110.4425) (end 137.65 110.43) (width 0.15) (layer "F.Cu") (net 10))
 (segment (start 148.185 110.83) (end 148.85 110.83) (width 0.15) (layer "F.Cu") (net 10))
 (segment (start 148.85 110.83) (end 149.25 110.43) (width 0.15) (layer "F.Cu") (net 10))
 (via (at 149.25 110.43) (size 0.6) (drill 0.3) (layers "F.Cu" "B.Cu") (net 10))
 (via (at 137.65 110.43) (size 0.6) (drill 0.3) (layers "F.Cu" "B.Cu") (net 10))
 (segment (start 149.25 110.43) (end 137.65 110.43) (width 0.15) (layer "B.Cu") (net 10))
 (segment (start 137.965 116.145) (end 137.965 116.63) (width 0.5) (layer "F.Cu") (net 12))
 (segment (start 137.6375 115.8175) (end 137.965 116.145) (width 0.5) (layer "F.Cu") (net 12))
 (segment (start 137.6375 115.085) (end 137.6375 115.8175) (width 0.5) (layer "F.Cu") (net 12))
 (segment (start 145.385 113.665) (end 145.95 114.23) (width 0.5) (layer "F.Cu") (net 6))
 (segment (start 144.95 113.665) (end 145.385 113.665) (width 0.5) (layer "F.Cu") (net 6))
 (segment (start 145.95 114.23) (end 146.715 114.23) (width 0.5) (layer "F.Cu") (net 6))
 (segment (start 144.065 113.815) (end 144.215 113.665) (width 0.5) (layer "F.Cu") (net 6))
 (segment (start 142.7625 113.815) (end 144.065 113.815) (width 0.5) (layer "F.Cu") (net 6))
 (segment (start 144.215 113.665) (end 144.95 113.665) (width 0.5) (layer "F.Cu") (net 6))
 (segment (start 145.935 115.33) (end 148.15 115.33) (width 0.15) (layer "F.Cu") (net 1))
 (segment (start 145.935 115.33) (end 145.935 116.43) (width 0.5) (layer "F.Cu") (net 1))
 (segment (start 146.6875 104.3675) (end 146.45 104.605) (width 0.15) (layer "F.Cu") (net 1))
 (segment (start 141.45 105.555) (end 141.45 103.43) (width 0.15) (layer "F.Cu") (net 1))
 (segment (start 138.8125 103.2925) (end 138.95 103.43) (width 0.15) (layer "F.Cu") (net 1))
 (segment (start 148.15 115.33) (end 150.92 112.56) (width 0.15) (layer "F.Cu") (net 1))
 (segment (start 150.92 112.56) (end 152.895 112.56) (width 0.15) (layer "F.Cu") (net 1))
 (segment (start 138.95 105.555) (end 138.95 103.43) (width 0.15) (layer "F.Cu") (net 1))
 (segment (start 141.45 105.555) (end 138.95 105.555) (width 0.15) (layer "F.Cu") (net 1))
 (segment (start 141.45 103.43) (end 138.95 103.43) (width 0.15) (layer "F.Cu") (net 1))
 (segment (start 147.685 113.13) (end 147.685 114.23) (width 0.5) (layer "F.Cu") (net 7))
 (segment (start 124.05 110.83) (end 124.05 113.48) (width 0.15) (layer "F.Cu") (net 5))
 (segment (start 124.05 116.23) (end 124.05 113.48) (width 0.15) (layer "F.Cu") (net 5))
 (segment (start 110.8375 102.83) (end 123.45 102.83) (width 0.15) (layer "F.Cu") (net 5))
 (segment (start 123.45 102.83) (end 124.05 103.43) (width 0.15) (layer "F.Cu") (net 5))
 (segment (start 137.565 112.6175) (end 137.6375 112.545) (width 0.15) (layer "F.Cu") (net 5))
 (segment (start 123.45 124.63) (end 124.05 124.03) (width 0.15) (layer "F.Cu") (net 5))
 (segment (start 115.55 124.63) (end 123.45 124.63) (width 0.15) (layer "F.Cu") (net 5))
 (via (at 124.05 124.03) (size 0.6) (drill 0.3) (layers "F.Cu" "B.Cu") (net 5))
 (via (at 124.05 103.43) (size 0.6) (drill 0.3) (layers "F.Cu" "B.Cu") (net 5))
 (via (at 124.05 116.23) (size 0.6) (drill 0.3) (layers "F.Cu" "B.Cu") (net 5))
 (via (at 124.05 110.83) (size 0.6) (drill 0.3) (layers "F.Cu" "B.Cu") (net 5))
 (segment (start 124.05 103.43) (end 124.05 110.83) (width 0.15) (layer "B.Cu") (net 5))
 (segment (start 124.05 124.03) (end 124.05 116.23) (width 0.15) (layer "B.Cu") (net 5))
 (segment (start 109.25 102.8425) (end 109.2625 102.83) (width 0.15) (layer "F.Cu") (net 8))
 (segment (start 109.25 104.21) (end 109.25 102.8425) (width 0.15) (layer "F.Cu") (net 8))
 (segment (start 135.45 127.03) (end 136.05 126.43) (width 0.15) (layer "F.Cu") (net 9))
 (segment (start 136.75 113.815) (end 137.6375 113.815) (width 0.15) (layer "F.Cu") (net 9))
 (segment (start 113.05 127.03) (end 135.45 127.03) (width 0.15) (layer "F.Cu") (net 9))
 (segment (start 136.05 114.515) (end 136.75 113.815) (width 0.15) (layer "F.Cu") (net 9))
 (via (at 136.05 126.43) (size 0.6) (drill 0.3) (layers "F.Cu" "B.Cu") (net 9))
 (via (at 136.05 114.515) (size 0.6) (drill 0.3) (layers "F.Cu" "B.Cu") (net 9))
 (segment (start 136.05 126.43) (end 136.05 114.515) (width 0.15) (layer "B.Cu") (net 9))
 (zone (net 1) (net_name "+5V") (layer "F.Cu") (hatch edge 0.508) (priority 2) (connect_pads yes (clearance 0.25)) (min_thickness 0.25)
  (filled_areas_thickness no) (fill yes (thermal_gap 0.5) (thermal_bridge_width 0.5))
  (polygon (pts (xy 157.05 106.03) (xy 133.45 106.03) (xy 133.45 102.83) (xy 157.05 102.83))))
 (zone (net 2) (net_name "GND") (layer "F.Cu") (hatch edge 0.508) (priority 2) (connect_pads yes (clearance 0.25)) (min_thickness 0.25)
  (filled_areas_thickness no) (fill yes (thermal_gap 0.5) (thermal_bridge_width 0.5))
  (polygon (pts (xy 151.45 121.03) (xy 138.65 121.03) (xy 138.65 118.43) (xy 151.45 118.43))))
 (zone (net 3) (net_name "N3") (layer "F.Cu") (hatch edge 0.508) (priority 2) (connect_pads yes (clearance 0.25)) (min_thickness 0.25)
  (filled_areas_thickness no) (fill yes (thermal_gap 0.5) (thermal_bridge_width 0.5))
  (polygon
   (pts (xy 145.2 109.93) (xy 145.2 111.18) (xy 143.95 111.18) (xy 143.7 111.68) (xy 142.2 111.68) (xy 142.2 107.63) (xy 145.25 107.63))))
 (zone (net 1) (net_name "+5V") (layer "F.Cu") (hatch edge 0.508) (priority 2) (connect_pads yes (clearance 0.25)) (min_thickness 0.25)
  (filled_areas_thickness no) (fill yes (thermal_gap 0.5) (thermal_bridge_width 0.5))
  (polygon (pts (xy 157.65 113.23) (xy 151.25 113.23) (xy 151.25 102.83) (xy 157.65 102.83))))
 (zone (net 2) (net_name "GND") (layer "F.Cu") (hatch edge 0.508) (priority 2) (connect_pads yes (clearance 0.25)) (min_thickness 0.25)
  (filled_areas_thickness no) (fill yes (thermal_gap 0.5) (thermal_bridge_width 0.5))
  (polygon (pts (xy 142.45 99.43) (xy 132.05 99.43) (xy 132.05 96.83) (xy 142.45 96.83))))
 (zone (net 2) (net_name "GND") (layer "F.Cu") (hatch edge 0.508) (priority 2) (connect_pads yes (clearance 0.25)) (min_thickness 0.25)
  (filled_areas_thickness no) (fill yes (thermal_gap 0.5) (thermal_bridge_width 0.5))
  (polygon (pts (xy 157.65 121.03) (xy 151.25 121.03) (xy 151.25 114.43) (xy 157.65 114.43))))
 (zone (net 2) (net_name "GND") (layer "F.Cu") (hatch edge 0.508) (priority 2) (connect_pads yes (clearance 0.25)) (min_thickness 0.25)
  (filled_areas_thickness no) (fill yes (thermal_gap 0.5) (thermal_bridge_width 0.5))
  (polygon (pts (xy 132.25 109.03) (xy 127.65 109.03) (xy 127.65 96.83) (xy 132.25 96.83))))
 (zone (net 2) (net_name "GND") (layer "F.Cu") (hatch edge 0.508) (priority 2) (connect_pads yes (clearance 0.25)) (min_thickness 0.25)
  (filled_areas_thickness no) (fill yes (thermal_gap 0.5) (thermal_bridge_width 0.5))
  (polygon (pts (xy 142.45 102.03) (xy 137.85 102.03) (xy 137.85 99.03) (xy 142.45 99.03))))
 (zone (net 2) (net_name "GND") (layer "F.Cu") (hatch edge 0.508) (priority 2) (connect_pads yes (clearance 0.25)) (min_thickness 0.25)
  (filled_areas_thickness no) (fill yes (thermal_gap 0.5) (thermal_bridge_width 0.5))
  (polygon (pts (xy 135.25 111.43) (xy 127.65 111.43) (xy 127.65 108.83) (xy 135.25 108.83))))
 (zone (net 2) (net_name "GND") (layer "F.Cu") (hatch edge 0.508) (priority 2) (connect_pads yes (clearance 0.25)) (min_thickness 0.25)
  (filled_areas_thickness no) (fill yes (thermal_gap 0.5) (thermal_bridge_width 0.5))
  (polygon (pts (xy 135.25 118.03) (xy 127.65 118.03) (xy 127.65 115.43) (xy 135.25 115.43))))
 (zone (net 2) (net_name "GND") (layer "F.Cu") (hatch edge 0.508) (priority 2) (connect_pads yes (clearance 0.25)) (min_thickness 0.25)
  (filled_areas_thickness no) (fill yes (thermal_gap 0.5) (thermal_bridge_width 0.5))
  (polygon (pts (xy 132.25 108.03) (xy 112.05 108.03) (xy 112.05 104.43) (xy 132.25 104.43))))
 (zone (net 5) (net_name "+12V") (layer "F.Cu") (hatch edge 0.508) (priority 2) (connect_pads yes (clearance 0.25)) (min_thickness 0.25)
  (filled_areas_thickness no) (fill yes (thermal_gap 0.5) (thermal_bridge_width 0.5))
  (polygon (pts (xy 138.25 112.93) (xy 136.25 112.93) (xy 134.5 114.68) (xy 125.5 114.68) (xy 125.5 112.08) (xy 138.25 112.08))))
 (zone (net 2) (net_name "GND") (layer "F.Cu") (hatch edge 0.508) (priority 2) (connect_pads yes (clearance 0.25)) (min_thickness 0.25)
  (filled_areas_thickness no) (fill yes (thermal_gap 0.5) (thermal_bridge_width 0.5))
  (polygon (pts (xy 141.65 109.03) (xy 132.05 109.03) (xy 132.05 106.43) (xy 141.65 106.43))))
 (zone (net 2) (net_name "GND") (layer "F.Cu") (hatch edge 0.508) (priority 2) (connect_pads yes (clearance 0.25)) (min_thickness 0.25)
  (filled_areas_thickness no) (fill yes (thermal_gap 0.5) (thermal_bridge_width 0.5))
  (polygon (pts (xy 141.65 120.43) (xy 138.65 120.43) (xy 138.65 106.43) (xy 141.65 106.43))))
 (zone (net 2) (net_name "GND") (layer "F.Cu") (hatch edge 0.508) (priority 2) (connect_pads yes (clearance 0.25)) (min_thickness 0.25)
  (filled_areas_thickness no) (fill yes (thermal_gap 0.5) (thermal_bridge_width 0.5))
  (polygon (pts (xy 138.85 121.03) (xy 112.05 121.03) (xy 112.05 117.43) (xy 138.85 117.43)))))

